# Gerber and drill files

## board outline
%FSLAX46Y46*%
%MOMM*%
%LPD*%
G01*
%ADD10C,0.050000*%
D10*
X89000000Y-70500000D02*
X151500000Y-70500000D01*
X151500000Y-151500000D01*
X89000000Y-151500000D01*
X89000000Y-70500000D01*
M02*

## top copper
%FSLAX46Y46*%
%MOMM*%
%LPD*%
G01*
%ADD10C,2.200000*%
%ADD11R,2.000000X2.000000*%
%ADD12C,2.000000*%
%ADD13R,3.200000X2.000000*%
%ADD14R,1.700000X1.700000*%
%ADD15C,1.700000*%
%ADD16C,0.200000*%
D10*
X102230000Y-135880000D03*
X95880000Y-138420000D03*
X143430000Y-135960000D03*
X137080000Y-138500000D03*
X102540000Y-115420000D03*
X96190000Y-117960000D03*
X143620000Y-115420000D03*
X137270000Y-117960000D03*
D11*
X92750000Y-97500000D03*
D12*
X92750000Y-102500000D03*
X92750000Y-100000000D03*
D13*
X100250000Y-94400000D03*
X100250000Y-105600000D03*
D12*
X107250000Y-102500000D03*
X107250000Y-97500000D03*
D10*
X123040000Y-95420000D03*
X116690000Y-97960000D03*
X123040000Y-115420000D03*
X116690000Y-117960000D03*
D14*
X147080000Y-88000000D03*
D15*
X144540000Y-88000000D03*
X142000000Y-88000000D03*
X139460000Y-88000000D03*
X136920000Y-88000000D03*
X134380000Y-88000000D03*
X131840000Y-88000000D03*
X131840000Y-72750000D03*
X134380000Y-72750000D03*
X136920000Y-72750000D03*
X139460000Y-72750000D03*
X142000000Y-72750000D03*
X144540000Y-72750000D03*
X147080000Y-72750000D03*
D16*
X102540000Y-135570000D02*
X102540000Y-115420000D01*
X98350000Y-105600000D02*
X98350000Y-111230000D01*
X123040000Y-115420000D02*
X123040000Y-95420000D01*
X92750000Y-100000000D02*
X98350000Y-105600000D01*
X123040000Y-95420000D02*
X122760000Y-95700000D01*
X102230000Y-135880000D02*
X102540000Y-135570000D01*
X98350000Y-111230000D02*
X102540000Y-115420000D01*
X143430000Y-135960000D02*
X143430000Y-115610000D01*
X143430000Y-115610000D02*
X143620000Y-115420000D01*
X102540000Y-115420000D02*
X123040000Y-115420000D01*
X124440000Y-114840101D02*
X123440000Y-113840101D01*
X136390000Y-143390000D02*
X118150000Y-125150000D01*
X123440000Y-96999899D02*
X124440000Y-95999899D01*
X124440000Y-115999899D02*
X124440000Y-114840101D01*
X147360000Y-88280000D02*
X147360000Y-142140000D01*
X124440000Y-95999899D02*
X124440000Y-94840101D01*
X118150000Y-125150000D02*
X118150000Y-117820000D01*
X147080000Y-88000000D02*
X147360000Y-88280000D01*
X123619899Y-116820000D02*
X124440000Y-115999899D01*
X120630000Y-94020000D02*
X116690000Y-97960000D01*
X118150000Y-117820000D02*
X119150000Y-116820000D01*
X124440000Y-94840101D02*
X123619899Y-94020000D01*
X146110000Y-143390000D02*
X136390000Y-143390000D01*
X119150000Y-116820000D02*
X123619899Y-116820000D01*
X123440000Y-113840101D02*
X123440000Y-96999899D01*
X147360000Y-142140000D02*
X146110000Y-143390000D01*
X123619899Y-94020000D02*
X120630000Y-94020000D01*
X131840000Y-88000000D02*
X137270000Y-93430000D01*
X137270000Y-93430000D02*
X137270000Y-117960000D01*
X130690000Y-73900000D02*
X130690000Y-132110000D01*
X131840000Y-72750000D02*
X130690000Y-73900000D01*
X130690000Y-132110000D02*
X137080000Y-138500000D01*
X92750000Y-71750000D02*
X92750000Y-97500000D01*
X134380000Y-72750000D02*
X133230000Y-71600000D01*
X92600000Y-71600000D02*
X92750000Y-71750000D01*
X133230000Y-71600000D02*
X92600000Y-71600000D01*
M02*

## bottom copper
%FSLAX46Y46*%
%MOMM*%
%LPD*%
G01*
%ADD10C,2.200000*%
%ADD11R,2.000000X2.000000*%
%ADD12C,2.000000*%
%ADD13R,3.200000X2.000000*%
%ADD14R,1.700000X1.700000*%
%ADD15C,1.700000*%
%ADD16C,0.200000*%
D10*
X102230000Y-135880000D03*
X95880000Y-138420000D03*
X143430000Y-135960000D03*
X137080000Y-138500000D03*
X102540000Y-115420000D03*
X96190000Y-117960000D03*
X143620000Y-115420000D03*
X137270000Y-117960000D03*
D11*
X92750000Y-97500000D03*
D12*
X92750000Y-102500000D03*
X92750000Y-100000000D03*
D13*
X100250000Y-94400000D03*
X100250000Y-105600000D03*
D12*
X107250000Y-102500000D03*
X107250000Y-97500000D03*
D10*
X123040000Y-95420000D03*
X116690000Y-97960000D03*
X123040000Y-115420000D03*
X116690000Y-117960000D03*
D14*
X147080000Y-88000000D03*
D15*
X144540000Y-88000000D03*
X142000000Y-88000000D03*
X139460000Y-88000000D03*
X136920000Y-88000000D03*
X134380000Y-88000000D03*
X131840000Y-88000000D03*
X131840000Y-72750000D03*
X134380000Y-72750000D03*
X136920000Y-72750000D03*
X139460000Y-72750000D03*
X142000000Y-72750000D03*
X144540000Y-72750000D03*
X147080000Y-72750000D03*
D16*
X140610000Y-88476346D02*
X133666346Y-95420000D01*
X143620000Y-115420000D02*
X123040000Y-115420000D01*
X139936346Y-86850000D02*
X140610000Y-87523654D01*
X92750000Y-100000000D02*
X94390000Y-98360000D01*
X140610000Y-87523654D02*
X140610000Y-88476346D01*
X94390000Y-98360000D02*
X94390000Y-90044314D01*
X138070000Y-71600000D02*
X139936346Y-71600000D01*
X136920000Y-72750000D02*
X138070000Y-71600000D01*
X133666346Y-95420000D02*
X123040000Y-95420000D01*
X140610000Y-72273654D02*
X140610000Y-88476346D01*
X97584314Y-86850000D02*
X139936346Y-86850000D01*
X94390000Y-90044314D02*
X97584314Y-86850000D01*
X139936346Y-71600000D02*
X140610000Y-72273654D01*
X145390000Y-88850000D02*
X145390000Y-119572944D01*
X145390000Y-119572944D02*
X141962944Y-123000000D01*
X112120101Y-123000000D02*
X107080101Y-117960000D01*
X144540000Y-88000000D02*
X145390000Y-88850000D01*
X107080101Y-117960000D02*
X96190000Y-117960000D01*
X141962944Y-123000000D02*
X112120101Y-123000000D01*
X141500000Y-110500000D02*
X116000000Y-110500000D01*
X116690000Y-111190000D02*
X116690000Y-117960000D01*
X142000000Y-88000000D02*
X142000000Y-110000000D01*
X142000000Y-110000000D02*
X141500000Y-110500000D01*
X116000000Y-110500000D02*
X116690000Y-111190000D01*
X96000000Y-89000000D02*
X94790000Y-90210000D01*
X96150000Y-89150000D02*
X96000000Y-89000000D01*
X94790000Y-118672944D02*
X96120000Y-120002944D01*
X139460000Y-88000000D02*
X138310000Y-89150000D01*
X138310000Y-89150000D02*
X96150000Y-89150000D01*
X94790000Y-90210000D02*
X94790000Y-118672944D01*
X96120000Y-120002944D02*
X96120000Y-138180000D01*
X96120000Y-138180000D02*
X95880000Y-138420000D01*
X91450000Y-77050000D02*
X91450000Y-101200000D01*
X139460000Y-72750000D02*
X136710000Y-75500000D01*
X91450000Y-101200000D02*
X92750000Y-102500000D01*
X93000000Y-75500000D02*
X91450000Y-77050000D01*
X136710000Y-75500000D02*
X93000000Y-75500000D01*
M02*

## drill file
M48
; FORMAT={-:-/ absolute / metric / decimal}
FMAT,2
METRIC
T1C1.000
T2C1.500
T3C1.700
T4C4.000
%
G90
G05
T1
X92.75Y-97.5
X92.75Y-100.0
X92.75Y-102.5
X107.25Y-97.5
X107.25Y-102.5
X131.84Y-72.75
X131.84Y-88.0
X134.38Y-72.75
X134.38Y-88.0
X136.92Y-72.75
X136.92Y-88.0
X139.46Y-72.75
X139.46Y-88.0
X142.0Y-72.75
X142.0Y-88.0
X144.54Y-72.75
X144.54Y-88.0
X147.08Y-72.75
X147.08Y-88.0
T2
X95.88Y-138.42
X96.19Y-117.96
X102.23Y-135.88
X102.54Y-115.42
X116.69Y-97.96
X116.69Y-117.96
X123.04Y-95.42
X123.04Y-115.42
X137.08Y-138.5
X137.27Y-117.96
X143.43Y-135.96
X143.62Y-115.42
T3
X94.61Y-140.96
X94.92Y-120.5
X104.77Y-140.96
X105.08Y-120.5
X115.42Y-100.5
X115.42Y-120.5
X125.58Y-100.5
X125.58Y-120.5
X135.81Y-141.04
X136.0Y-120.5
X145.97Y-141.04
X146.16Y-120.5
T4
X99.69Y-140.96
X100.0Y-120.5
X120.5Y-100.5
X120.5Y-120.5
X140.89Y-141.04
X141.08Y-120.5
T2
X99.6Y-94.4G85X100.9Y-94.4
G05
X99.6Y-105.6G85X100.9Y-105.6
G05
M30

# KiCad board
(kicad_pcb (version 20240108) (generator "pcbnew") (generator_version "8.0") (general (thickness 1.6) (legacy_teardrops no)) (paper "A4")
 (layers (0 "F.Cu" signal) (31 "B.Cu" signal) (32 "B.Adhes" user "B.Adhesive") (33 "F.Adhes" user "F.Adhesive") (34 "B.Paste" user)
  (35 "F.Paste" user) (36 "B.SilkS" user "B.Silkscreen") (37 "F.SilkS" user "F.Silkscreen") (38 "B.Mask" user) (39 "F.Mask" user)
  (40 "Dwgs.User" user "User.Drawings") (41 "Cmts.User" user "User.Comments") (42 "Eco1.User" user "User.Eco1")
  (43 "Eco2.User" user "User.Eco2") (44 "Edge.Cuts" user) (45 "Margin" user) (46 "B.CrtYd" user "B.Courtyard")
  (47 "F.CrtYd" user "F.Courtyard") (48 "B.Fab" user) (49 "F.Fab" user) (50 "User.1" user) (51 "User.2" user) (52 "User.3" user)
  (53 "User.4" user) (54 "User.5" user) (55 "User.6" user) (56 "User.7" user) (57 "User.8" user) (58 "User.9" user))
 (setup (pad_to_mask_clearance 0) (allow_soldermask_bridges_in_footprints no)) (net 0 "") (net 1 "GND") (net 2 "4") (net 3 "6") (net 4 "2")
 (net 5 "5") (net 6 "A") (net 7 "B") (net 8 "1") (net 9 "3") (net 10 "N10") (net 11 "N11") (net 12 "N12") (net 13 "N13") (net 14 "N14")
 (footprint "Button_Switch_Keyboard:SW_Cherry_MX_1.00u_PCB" (layer "F.Cu") (at 102.23 135.88)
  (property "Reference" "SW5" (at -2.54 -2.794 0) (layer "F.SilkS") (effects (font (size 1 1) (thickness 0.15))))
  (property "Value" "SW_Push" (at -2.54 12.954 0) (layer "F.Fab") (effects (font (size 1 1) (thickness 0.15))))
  (pad "" np_thru_hole circle (at -7.62 5.08) (size 1.7 1.7) (drill 1.7) (layers "*.Cu" "*.Mask"))
  (pad "" np_thru_hole circle (at -2.54 5.08) (size 4 4) (drill 4) (layers "*.Cu" "*.Mask"))
  (pad "" np_thru_hole circle (at 2.54 5.08) (size 1.7 1.7) (drill 1.7) (layers "*.Cu" "*.Mask"))
  (pad "1" thru_hole circle (at 0 0) (size 2.2 2.2) (drill 1.5) (layers "*.Cu" "*.Mask") (remove_unused_layers no) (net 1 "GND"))
  (pad "2" thru_hole circle (at -6.35 2.54) (size 2.2 2.2) (drill 1.5) (layers "*.Cu" "*.Mask") (remove_unused_layers no) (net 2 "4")))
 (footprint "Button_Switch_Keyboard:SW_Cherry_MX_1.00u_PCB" (layer "F.Cu") (at 143.43 135.96)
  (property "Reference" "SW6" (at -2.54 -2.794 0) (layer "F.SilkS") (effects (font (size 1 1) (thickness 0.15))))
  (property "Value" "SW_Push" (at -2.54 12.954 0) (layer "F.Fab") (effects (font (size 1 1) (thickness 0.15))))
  (pad "" np_thru_hole circle (at -7.62 5.08) (size 1.7 1.7) (drill 1.7) (layers "*.Cu" "*.Mask"))
  (pad "" np_thru_hole circle (at -2.54 5.08) (size 4 4) (drill 4) (layers "*.Cu" "*.Mask"))
  (pad "" np_thru_hole circle (at 2.54 5.08) (size 1.7 1.7) (drill 1.7) (layers "*.Cu" "*.Mask"))
  (pad "1" thru_hole circle (at 0 0) (size 2.2 2.2) (drill 1.5) (layers "*.Cu" "*.Mask") (remove_unused_layers no) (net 1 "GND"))
  (pad "2" thru_hole circle (at -6.35 2.54) (size 2.2 2.2) (drill 1.5) (layers "*.Cu" "*.Mask") (remove_unused_layers no) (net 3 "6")))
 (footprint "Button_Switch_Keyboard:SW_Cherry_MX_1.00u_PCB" (layer "F.Cu") (at 102.54 115.42)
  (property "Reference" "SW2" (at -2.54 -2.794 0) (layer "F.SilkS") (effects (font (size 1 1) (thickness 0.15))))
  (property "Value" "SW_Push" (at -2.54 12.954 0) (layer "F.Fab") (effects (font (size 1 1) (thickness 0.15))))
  (pad "" np_thru_hole circle (at -7.62 5.08) (size 1.7 1.7) (drill 1.7) (layers "*.Cu" "*.Mask"))
  (pad "" np_thru_hole circle (at -2.54 5.08) (size 4 4) (drill 4) (layers "*.Cu" "*.Mask"))
  (pad "" np_thru_hole circle (at 2.54 5.08) (size 1.7 1.7) (drill 1.7) (layers "*.Cu" "*.Mask"))
  (pad "1" thru_hole circle (at 0 0) (size 2.2 2.2) (drill 1.5) (layers "*.Cu" "*.Mask") (remove_unused_layers no) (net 1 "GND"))
  (pad "2" thru_hole circle (at -6.35 2.54) (size 2.2 2.2) (drill 1.5) (layers "*.Cu" "*.Mask") (remove_unused_layers no) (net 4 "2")))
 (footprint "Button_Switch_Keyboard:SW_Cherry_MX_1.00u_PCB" (layer "F.Cu") (at 143.62 115.42)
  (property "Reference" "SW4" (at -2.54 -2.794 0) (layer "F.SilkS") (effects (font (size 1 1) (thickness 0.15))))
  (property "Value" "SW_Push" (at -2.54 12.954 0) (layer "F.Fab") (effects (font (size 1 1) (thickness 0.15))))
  (pad "" np_thru_hole circle (at -7.62 5.08) (size 1.7 1.7) (drill 1.7) (layers "*.Cu" "*.Mask"))
  (pad "" np_thru_hole circle (at -2.54 5.08) (size 4 4) (drill 4) (layers "*.Cu" "*.Mask"))
  (pad "" np_thru_hole circle (at 2.54 5.08) (size 1.7 1.7) (drill 1.7) (layers "*.Cu" "*.Mask"))
  (pad "1" thru_hole circle (at 0 0) (size 2.2 2.2) (drill 1.5) (layers "*.Cu" "*.Mask") (remove_unused_layers no) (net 1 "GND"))
  (pad "2" thru_hole circle (at -6.35 2.54) (size 2.2 2.2) (drill 1.5) (layers "*.Cu" "*.Mask") (remove_unused_layers no) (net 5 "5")))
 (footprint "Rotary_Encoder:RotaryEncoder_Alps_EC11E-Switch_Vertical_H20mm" (layer "F.Cu") (at 92.75 97.5)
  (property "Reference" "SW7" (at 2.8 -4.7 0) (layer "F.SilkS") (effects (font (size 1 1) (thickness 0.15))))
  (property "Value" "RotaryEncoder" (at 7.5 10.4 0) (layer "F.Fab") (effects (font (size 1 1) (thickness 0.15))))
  (pad "A" thru_hole rect (at 0 0) (size 2 2) (drill 1) (layers "*.Cu" "*.Mask") (remove_unused_layers no) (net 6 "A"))
  (pad "B" thru_hole circle (at 0 5) (size 2 2) (drill 1) (layers "*.Cu" "*.Mask") (remove_unused_layers no) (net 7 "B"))
  (pad "C" thru_hole circle (at 0 2.5) (size 2 2) (drill 1) (layers "*.Cu" "*.Mask") (remove_unused_layers no) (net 1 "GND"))
  (pad "MP" thru_hole rect (at 7.5 -3.1) (size 3.2 2) (drill oval 2.8 1.5) (layers "*.Cu" "*.Mask") (remove_unused_layers no))
  (pad "MP" thru_hole rect (at 7.5 8.1) (size 3.2 2) (drill oval 2.8 1.5) (layers "*.Cu" "*.Mask") (remove_unused_layers no))
  (pad "S1" thru_hole circle (at 14.5 5) (size 2 2) (drill 1) (layers "*.Cu" "*.Mask") (remove_unused_layers no))
  (pad "S2" thru_hole circle (at 14.5 0) (size 2 2) (drill 1) (layers "*.Cu" "*.Mask") (remove_unused_layers no)))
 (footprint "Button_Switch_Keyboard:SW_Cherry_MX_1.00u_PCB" (layer "F.Cu") (at 123.04 95.42)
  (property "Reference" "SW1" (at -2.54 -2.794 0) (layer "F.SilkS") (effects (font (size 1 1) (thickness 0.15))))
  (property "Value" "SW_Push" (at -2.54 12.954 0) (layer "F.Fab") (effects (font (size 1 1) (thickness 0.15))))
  (pad "" np_thru_hole circle (at -7.62 5.08) (size 1.7 1.7) (drill 1.7) (layers "*.Cu" "*.Mask"))
  (pad "" np_thru_hole circle (at -2.54 5.08) (size 4 4) (drill 4) (layers "*.Cu" "*.Mask"))
  (pad "" np_thru_hole circle (at 2.54 5.08) (size 1.7 1.7) (drill 1.7) (layers "*.Cu" "*.Mask"))
  (pad "1" thru_hole circle (at 0 0) (size 2.2 2.2) (drill 1.5) (layers "*.Cu" "*.Mask") (remove_unused_layers no) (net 1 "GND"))
  (pad "2" thru_hole circle (at -6.35 2.54) (size 2.2 2.2) (drill 1.5) (layers "*.Cu" "*.Mask") (remove_unused_layers no) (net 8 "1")))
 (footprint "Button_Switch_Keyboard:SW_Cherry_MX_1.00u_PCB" (layer "F.Cu") (at 123.04 115.42)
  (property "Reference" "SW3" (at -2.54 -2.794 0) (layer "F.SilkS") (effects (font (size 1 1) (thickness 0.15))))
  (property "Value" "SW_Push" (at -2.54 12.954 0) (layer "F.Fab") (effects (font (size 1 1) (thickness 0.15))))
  (pad "" np_thru_hole circle (at -7.62 5.08) (size 1.7 1.7) (drill 1.7) (layers "*.Cu" "*.Mask"))
  (pad "" np_thru_hole circle (at -2.54 5.08) (size 4 4) (drill 4) (layers "*.Cu" "*.Mask"))
  (pad "" np_thru_hole circle (at 2.54 5.08) (size 1.7 1.7) (drill 1.7) (layers "*.Cu" "*.Mask"))
  (pad "1" thru_hole circle (at 0 0) (size 2.2 2.2) (drill 1.5) (layers "*.Cu" "*.Mask") (remove_unused_layers no) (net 1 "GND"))
  (pad "2" thru_hole circle (at -6.35 2.54) (size 2.2 2.2) (drill 1.5) (layers "*.Cu" "*.Mask") (remove_unused_layers no) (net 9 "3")))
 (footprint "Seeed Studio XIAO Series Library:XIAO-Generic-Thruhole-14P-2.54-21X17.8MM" (layer "B.Cu") (at 139.46 80.375 90)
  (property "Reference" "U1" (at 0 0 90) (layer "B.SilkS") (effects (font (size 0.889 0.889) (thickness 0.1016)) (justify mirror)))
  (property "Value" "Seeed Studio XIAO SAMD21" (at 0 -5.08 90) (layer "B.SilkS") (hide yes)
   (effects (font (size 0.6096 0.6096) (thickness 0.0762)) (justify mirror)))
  (pad "1" thru_hole rect (at -7.625 7.62 90) (size 1.7 1.7) (drill 1) (layers "*.Cu" "*.Mask") (remove_unused_layers no) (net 8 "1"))
  (pad "2" thru_hole circle (at -7.625 5.08 90) (size 1.7 1.7) (drill 1) (layers "*.Cu" "*.Mask") (remove_unused_layers no) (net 4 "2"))
  (pad "3" thru_hole circle (at -7.625 2.54 90) (size 1.7 1.7) (drill 1) (layers "*.Cu" "*.Mask") (remove_unused_layers no) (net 9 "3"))
  (pad "4" thru_hole circle (at -7.625 0 90) (size 1.7 1.7) (drill 1) (layers "*.Cu" "*.Mask") (remove_unused_layers no) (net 2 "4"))
  (pad "5" thru_hole circle (at -7.625 -2.54 90) (size 1.7 1.7) (drill 1) (layers "*.Cu" "*.Mask") (remove_unused_layers no) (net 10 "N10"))
  (pad "6" thru_hole circle (at -7.625 -5.08 270) (size 1.7 1.7) (drill 1) (layers "*.Cu" "*.Mask") (remove_unused_layers no) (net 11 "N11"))
  (pad "7" thru_hole circle (at -7.625 -7.62 90) (size 1.7 1.7) (drill 1) (layers "*.Cu" "*.Mask") (remove_unused_layers no) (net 5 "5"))
  (pad "8" thru_hole circle (at 7.625 -7.62 90) (size 1.7 1.7) (drill 1) (layers "*.Cu" "*.Mask") (remove_unused_layers no) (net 3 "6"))
  (pad "9" thru_hole circle (at 7.625 -5.08 90) (size 1.7 1.7) (drill 1) (layers "*.Cu" "*.Mask") (remove_unused_layers no) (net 6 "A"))
  (pad "10" thru_hole circle (at 7.625 -2.54 90) (size 1.7 1.7) (drill 1) (layers "*.Cu" "*.Mask") (remove_unused_layers no) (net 1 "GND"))
  (pad "11" thru_hole circle (at 7.625 0 90) (size 1.7 1.7) (drill 1) (layers "*.Cu" "*.Mask") (remove_unused_layers no) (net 7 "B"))
  (pad "12" thru_hole circle (at 7.625 2.54 90) (size 1.7 1.7) (drill 1) (layers "*.Cu" "*.Mask") (remove_unused_layers no) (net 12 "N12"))
  (pad "13" thru_hole circle (at 7.625 5.08 90) (size 1.7 1.7) (drill 1) (layers "*.Cu" "*.Mask") (remove_unused_layers no) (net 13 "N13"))
  (pad "14" thru_hole circle (at 7.625 7.62 90) (size 1.7 1.7) (drill 1) (layers "*.Cu" "*.Mask") (remove_unused_layers no) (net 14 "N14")))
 (gr_rect (start 89 70.5) (end 151.5 151.5) (stroke (width 0.05) (type default)) (fill none) (layer "Edge.Cuts"))
 (segment (start 102.54 135.57) (end 102.54 115.42) (width 0.2) (layer "F.Cu") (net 1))
 (segment (start 98.35 105.6) (end 98.35 111.23) (width 0.2) (layer "F.Cu") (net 1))
 (segment (start 123.04 115.42) (end 123.04 95.42) (width 0.2) (layer "F.Cu") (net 1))
 (segment (start 92.75 100) (end 98.35 105.6) (width 0.2) (layer "F.Cu") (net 1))
 (segment (start 123.04 95.42) (end 122.76 95.7) (width 0.2) (layer "F.Cu") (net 1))
 (segment (start 102.23 135.88) (end 102.54 135.57) (width 0.2) (layer "F.Cu") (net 1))
 (segment (start 98.35 111.23) (end 102.54 115.42) (width 0.2) (layer "F.Cu") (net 1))
 (segment (start 143.43 135.96) (end 143.43 115.61) (width 0.2) (layer "F.Cu") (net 1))
 (segment (start 143.43 115.61) (end 143.62 115.42) (width 0.2) (layer "F.Cu") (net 1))
 (segment (start 102.54 115.42) (end 123.04 115.42) (width 0.2) (layer "F.Cu") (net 1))
 (segment (start 140.61 88.476346) (end 133.666346 95.42) (width 0.2) (layer "B.Cu") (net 1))
 (segment (start 143.62 115.42) (end 123.04 115.42) (width 0.2) (layer "B.Cu") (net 1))
 (segment (start 139.936346 86.85) (end 140.61 87.523654) (width 0.2) (layer "B.Cu") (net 1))
 (segment (start 92.75 100) (end 94.39 98.36) (width 0.2) (layer "B.Cu") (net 1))
 (segment (start 140.61 87.523654) (end 140.61 88.476346) (width 0.2) (layer "B.Cu") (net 1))
 (segment (start 94.39 98.36) (end 94.39 90.044314) (width 0.2) (layer "B.Cu") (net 1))
 (segment (start 138.07 71.6) (end 139.936346 71.6) (width 0.2) (layer "B.Cu") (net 1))
 (segment (start 136.92 72.75) (end 138.07 71.6) (width 0.2) (layer "B.Cu") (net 1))
 (segment (start 133.666346 95.42) (end 123.04 95.42) (width 0.2) (layer "B.Cu") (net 1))
 (segment (start 140.61 72.273654) (end 140.61 88.476346) (width 0.2) (layer "B.Cu") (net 1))
 (segment (start 97.584314 86.85) (end 139.936346 86.85) (width 0.2) (layer "B.Cu") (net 1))
 (segment (start 94.39 90.044314) (end 97.584314 86.85) (width 0.2) (layer "B.Cu") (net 1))
 (segment (start 139.936346 71.6) (end 140.61 72.273654) (width 0.2) (layer "B.Cu") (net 1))
 (segment (start 124.44 114.840101) (end 123.44 113.840101) (width 0.2) (layer "F.Cu") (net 8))
 (segment (start 136.39 143.39) (end 118.15 125.15) (width 0.2) (layer "F.Cu") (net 8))
 (segment (start 123.44 96.999899) (end 124.44 95.999899) (width 0.2) (layer "F.Cu") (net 8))
 (segment (start 124.44 115.999899) (end 124.44 114.840101) (width 0.2) (layer "F.Cu") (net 8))
 (segment (start 147.36 88.28) (end 147.36 142.14) (width 0.2) (layer "F.Cu") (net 8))
 (segment (start 124.44 95.999899) (end 124.44 94.840101) (width 0.2) (layer "F.Cu") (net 8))
 (segment (start 118.15 125.15) (end 118.15 117.82) (width 0.2) (layer "F.Cu") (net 8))
 (segment (start 147.08 88) (end 147.36 88.28) (width 0.2) (layer "F.Cu") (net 8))
 (segment (start 123.619899 116.82) (end 124.44 115.999899) (width 0.2) (layer "F.Cu") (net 8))
 (segment (start 120.63 94.02) (end 116.69 97.96) (width 0.2) (layer "F.Cu") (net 8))
 (segment (start 118.15 117.82) (end 119.15 116.82) (width 0.2) (layer "F.Cu") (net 8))
 (segment (start 124.44 94.840101) (end 123.619899 94.02) (width 0.2) (layer "F.Cu") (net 8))
 (segment (start 146.11 143.39) (end 136.39 143.39) (width 0.2) (layer "F.Cu") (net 8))
 (segment (start 119.15 116.82) (end 123.619899 116.82) (width 0.2) (layer "F.Cu") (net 8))
 (segment (start 123.44 113.840101) (end 123.44 96.999899) (width 0.2) (layer "F.Cu") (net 8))
 (segment (start 147.36 142.14) (end 146.11 143.39) (width 0.2) (layer "F.Cu") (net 8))
 (segment (start 123.619899 94.02) (end 120.63 94.02) (width 0.2) (layer "F.Cu") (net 8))
 (segment (start 145.39 88.85) (end 145.39 119.572944) (width 0.2) (layer "B.Cu") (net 4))
 (segment (start 145.39 119.572944) (end 141.962944 123) (width 0.2) (layer "B.Cu") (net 4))
 (segment (start 112.120101 123) (end 107.080101 117.96) (width 0.2) (layer "B.Cu") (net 4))
 (segment (start 144.54 88) (end 145.39 88.85) (width 0.2) (layer "B.Cu") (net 4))
 (segment (start 107.080101 117.96) (end 96.19 117.96) (width 0.2) (layer "B.Cu") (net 4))
 (segment (start 141.962944 123) (end 112.120101 123) (width 0.2) (layer "B.Cu") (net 4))
 (segment (start 141.5 110.5) (end 116 110.5) (width 0.2) (layer "B.Cu") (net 9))
 (segment (start 116.69 111.19) (end 116.69 117.96) (width 0.2) (layer "B.Cu") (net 9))
 (segment (start 142 88) (end 142 110) (width 0.2) (layer "B.Cu") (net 9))
 (segment (start 142 110) (end 141.5 110.5) (width 0.2) (layer "B.Cu") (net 9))
 (segment (start 116 110.5) (end 116.69 111.19) (width 0.2) (layer "B.Cu") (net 9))
 (segment (start 131.84 88) (end 137.27 93.43) (width 0.2) (layer "F.Cu") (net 5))
 (segment (start 137.27 93.43) (end 137.27 117.96) (width 0.2) (layer "F.Cu") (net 5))
 (segment (start 96 89) (end 94.79 90.21) (width 0.2) (layer "B.Cu") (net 2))
 (segment (start 96.15 89.15) (end 96 89) (width 0.2) (layer "B.Cu") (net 2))
 (segment (start 94.79 118.672944) (end 96.12 120.002944) (width 0.2) (layer "B.Cu") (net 2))
 (segment (start 139.46 88) (end 138.31 89.15) (width 0.2) (layer "B.Cu") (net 2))
 (segment (start 138.31 89.15) (end 96.15 89.15) (width 0.2) (layer "B.Cu") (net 2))
 (segment (start 94.79 90.21) (end 94.79 118.672944) (width 0.2) (layer "B.Cu") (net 2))
 (segment (start 96.12 120.002944) (end 96.12 138.18) (width 0.2) (layer "B.Cu") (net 2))
 (segment (start 96.12 138.18) (end 95.88 138.42) (width 0.2) (layer "B.Cu") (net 2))
 (segment (start 130.69 73.9) (end 130.69 132.11) (width 0.2) (layer "F.Cu") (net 3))
 (segment (start 131.84 72.75) (end 130.69 73.9) (width 0.2) (layer "F.Cu") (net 3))
 (segment (start 130.69 132.11) (end 137.08 138.5) (width 0.2) (layer "F.Cu") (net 3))
 (segment (start 91.45 77.05) (end 91.45 101.2) (width 0.2) (layer "B.Cu") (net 7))
 (segment (start 139.46 72.75) (end 136.71 75.5) (width 0.2) (layer "B.Cu") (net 7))
 (segment (start 91.45 101.2) (end 92.75 102.5) (width 0.2) (layer "B.Cu") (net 7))
 (segment (start 93 75.5) (end 91.45 77.05) (width 0.2) (layer "B.Cu") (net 7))
 (segment (start 136.71 75.5) (end 93 75.5) (width 0.2) (layer "B.Cu") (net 7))
 (segment (start 92.75 71.75) (end 92.75 97.5) (width 0.2) (layer "F.Cu") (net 6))
 (segment (start 134.38 72.75) (end 133.23 71.6) (width 0.2) (layer "F.Cu") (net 6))
 (segment (start 92.6 71.6) (end 92.75 71.75) (width 0.2) (layer "F.Cu") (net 6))
 (segment (start 133.23 71.6) (end 92.6 71.6) (width 0.2) (layer "F.Cu") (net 6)))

